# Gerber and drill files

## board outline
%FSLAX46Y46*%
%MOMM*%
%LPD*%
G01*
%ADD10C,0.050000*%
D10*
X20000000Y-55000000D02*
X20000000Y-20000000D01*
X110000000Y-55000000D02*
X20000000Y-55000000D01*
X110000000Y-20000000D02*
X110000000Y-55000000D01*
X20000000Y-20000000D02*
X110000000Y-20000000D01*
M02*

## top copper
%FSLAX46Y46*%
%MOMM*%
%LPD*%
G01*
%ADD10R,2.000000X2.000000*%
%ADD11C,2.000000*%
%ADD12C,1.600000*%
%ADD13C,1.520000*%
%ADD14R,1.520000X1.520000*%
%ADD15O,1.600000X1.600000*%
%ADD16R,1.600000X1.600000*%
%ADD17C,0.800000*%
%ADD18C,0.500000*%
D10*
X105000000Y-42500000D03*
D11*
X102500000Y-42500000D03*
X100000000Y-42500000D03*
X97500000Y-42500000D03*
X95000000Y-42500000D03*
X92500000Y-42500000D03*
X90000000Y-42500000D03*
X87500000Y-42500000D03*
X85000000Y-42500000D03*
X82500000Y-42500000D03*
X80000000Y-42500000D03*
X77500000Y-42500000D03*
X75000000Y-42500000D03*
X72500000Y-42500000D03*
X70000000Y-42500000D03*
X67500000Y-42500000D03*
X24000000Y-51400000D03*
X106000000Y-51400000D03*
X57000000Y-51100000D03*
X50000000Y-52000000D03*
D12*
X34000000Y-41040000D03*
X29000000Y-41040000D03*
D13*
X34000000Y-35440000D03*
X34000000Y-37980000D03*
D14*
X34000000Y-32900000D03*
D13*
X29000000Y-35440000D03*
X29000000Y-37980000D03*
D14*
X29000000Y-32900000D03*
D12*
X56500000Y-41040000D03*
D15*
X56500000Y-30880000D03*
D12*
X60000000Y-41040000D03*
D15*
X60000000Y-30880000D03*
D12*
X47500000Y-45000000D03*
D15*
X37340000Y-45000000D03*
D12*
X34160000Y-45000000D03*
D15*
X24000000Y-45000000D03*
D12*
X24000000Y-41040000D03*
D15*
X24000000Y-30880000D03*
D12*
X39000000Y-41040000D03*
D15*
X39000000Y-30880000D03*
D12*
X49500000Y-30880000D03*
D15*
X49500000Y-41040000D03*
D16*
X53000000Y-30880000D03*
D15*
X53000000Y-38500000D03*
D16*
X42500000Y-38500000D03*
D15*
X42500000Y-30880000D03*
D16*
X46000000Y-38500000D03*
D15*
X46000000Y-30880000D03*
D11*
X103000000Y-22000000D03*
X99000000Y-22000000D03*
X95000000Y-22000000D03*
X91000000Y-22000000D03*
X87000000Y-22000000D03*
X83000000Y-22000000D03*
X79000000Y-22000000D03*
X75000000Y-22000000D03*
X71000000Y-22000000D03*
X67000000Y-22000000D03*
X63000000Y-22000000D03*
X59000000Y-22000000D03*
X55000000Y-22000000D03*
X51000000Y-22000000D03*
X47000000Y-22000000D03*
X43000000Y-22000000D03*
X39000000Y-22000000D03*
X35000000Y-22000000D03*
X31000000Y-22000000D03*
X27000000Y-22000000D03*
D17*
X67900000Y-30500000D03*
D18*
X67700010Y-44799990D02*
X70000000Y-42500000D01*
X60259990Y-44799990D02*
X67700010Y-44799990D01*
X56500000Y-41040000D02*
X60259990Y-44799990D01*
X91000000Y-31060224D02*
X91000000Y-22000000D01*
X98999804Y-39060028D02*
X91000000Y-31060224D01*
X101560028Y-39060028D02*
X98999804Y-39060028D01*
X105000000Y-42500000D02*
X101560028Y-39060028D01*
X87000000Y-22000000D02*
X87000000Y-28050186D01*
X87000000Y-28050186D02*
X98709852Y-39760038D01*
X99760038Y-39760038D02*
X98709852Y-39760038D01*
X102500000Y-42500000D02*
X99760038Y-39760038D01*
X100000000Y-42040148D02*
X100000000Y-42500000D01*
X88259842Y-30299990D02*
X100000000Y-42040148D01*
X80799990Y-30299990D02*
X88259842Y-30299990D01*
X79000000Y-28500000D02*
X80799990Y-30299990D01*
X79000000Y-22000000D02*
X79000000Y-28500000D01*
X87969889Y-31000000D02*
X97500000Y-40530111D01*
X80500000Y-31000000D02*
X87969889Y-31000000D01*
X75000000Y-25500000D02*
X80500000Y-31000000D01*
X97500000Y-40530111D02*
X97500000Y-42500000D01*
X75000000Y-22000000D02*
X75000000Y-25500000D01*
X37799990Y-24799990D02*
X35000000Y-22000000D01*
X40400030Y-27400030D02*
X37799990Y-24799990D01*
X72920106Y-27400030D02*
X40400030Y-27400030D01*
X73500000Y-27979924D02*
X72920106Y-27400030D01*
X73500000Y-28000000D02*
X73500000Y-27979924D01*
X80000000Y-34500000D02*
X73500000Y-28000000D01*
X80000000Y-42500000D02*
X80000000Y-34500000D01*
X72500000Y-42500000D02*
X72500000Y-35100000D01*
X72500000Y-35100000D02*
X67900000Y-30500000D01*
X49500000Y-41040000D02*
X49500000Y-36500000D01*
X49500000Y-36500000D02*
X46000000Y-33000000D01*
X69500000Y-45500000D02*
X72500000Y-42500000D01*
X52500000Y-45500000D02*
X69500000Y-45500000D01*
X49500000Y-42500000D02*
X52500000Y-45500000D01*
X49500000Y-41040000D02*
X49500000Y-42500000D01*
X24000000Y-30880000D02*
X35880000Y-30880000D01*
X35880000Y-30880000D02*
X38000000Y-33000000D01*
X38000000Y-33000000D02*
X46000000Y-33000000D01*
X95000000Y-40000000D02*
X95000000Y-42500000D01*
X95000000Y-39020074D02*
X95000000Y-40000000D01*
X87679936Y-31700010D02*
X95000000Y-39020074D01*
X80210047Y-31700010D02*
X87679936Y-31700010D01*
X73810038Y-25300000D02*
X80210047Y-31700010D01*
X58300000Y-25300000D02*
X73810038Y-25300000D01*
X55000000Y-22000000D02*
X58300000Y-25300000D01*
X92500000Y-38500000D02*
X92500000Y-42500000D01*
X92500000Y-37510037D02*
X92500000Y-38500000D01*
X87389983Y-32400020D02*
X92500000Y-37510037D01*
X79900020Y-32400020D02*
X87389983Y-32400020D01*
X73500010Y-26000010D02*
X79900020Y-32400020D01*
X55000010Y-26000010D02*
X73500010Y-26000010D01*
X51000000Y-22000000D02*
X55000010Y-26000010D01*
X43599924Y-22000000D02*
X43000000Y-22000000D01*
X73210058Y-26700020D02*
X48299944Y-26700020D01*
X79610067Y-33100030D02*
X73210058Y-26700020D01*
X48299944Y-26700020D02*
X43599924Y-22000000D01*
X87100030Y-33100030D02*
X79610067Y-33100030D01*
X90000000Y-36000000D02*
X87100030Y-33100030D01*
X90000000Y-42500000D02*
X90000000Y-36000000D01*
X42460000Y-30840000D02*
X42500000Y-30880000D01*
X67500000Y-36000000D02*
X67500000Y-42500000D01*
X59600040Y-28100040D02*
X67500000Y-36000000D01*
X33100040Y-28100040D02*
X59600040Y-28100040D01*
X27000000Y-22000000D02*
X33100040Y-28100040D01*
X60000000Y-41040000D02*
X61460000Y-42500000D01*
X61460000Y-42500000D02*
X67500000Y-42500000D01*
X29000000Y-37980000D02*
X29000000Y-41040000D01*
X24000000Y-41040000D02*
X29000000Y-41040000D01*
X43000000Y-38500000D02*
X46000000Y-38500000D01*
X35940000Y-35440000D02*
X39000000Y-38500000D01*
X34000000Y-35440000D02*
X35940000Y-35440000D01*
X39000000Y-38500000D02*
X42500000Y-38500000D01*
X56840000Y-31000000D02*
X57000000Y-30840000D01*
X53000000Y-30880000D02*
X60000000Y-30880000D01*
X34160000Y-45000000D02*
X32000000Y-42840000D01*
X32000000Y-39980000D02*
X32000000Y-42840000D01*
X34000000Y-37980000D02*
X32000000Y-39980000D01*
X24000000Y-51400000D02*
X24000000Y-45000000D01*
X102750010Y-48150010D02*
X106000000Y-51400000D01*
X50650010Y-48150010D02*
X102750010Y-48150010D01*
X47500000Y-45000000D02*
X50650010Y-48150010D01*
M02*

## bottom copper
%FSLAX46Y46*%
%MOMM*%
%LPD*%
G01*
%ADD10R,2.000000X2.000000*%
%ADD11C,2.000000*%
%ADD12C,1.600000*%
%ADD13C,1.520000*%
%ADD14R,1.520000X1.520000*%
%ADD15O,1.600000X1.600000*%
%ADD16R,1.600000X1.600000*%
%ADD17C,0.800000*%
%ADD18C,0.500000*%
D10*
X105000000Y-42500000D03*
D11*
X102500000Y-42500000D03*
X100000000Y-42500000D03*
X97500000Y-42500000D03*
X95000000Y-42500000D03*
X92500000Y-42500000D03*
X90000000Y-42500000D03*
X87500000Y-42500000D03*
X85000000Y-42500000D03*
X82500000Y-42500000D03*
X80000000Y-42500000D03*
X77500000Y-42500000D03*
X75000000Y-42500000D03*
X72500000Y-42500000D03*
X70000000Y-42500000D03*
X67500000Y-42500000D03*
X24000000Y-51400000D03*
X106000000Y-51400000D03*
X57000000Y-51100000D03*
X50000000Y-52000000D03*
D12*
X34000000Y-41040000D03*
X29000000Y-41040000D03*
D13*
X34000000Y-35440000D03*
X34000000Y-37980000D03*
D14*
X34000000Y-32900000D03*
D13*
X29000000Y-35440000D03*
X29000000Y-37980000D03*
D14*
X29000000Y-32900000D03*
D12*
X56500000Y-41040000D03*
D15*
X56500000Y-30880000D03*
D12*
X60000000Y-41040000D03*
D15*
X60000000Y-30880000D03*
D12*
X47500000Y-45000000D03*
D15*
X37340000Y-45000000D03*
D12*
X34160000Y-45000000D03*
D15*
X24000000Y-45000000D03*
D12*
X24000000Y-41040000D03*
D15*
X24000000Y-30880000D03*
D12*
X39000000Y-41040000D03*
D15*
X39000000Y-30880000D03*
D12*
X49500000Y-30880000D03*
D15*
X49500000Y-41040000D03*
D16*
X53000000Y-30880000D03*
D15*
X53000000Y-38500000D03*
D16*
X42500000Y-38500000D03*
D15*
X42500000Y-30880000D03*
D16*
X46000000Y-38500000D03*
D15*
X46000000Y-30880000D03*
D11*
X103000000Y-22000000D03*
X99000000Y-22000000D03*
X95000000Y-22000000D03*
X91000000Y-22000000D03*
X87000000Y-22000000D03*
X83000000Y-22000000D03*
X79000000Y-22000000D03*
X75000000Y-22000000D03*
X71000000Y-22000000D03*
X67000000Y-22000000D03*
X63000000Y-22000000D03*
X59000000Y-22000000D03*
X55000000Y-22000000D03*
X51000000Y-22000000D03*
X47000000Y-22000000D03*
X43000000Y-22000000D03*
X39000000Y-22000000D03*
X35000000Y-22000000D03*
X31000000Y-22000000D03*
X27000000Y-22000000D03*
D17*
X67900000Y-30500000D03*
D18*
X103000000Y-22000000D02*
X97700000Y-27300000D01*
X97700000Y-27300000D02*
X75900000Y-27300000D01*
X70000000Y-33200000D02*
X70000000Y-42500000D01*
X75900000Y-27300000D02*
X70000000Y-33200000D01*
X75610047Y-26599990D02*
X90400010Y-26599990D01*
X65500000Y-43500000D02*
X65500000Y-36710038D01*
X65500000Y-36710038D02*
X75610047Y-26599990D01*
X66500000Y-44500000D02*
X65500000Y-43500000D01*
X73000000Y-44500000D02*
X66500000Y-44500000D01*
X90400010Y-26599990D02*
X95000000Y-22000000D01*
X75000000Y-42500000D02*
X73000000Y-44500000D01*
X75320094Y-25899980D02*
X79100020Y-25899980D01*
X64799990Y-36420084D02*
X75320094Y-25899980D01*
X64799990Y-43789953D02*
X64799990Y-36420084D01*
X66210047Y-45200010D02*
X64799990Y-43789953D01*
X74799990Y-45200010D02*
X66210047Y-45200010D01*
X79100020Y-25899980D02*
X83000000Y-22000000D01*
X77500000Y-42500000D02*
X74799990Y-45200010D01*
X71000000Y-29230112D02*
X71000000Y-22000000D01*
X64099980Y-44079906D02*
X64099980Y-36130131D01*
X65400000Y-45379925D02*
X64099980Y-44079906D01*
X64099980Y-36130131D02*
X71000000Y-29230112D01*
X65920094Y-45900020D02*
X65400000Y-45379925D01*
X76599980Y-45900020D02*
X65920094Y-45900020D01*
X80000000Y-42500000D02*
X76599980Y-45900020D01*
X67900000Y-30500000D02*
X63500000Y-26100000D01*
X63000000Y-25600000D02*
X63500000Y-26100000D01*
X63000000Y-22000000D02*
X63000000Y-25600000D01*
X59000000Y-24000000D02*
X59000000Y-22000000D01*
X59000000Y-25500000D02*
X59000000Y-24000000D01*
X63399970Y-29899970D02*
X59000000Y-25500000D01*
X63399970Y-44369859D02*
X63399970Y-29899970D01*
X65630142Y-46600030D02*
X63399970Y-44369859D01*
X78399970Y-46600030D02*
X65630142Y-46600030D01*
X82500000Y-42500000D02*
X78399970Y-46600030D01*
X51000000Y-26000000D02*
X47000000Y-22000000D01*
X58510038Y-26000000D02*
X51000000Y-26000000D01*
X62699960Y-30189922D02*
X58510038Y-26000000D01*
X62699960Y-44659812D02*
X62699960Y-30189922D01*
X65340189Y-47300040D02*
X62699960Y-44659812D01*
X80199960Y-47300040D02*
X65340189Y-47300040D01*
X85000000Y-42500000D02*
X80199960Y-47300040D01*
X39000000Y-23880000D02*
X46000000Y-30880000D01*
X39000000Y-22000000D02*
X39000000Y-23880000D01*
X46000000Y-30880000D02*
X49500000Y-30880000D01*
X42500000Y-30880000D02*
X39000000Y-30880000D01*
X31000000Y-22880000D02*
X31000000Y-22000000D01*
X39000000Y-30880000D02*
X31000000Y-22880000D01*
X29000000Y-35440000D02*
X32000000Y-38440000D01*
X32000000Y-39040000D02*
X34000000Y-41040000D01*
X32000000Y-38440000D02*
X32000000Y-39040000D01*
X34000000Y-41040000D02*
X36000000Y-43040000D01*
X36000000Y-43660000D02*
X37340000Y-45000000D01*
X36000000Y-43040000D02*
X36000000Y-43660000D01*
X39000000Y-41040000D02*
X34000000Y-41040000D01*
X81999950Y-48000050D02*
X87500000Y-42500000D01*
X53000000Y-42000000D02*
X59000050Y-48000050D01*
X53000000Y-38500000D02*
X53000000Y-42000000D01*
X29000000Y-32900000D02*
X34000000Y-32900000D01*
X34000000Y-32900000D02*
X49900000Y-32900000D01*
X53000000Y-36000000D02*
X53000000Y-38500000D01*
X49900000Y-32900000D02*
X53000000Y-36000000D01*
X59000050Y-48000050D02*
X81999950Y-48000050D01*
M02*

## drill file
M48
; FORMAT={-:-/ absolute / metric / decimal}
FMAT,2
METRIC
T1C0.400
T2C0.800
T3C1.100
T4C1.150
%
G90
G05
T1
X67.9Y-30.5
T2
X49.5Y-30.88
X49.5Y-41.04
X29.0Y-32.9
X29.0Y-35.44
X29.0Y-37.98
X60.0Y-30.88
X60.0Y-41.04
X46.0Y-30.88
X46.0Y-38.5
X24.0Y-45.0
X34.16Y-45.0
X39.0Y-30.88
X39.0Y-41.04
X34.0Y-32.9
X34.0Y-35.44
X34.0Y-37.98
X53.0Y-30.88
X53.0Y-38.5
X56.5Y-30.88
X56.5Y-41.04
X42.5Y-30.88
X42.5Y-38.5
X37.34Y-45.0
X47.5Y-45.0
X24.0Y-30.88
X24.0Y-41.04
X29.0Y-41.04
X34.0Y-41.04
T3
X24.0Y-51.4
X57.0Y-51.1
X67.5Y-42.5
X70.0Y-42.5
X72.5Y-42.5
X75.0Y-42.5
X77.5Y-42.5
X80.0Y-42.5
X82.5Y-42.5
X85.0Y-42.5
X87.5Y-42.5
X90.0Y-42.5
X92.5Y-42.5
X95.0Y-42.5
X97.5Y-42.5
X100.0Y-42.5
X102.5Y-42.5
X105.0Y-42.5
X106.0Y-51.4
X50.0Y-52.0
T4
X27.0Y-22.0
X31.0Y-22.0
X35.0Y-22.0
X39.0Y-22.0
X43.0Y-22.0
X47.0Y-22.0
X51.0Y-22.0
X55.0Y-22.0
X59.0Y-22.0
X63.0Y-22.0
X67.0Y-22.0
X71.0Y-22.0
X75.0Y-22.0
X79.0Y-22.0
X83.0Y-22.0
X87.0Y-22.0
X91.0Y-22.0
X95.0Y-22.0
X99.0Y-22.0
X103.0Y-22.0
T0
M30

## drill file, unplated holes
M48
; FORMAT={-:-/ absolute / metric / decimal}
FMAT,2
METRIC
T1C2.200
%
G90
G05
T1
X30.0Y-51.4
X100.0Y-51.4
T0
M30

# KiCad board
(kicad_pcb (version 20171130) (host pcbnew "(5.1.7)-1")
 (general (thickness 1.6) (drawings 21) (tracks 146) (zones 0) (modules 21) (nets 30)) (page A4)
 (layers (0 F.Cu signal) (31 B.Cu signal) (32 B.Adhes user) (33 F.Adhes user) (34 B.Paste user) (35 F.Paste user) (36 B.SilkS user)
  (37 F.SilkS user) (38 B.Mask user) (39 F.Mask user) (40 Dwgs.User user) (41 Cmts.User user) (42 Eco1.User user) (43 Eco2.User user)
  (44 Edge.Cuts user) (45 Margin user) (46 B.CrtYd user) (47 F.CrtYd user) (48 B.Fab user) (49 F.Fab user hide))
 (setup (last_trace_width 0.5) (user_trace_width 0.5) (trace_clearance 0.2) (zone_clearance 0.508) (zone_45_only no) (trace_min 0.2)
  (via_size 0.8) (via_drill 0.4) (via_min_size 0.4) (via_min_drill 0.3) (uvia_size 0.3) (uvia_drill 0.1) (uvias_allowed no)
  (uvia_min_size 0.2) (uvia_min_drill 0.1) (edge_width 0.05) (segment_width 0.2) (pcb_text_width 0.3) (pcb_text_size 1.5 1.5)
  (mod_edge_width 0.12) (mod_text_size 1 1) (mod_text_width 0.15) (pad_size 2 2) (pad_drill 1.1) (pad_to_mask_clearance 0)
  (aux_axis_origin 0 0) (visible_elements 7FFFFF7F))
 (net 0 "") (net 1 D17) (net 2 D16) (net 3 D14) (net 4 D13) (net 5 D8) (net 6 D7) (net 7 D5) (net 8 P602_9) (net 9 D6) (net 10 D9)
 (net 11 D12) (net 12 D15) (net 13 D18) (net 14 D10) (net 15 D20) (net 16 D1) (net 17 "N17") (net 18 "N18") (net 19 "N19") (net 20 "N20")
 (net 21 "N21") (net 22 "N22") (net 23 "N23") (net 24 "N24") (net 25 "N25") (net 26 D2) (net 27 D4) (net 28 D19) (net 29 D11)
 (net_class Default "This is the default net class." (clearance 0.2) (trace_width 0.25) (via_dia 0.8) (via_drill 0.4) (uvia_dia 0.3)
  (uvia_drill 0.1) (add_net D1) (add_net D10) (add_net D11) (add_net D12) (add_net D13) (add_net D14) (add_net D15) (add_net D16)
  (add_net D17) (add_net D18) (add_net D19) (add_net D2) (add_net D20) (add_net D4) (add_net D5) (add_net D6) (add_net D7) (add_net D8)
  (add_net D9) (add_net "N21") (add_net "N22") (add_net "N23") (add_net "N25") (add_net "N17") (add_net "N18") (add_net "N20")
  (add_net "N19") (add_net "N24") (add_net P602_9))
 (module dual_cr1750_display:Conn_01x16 (layer F.Cu) (at 105 42.5 180) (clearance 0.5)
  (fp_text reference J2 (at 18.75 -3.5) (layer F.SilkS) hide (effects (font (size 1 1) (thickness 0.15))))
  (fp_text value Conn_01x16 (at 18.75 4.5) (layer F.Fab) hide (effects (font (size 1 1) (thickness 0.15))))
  (pad 1 thru_hole rect (at 0 0 180) (size 2 2) (drill 1.1) (layers *.Cu *.Mask) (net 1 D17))
  (pad 2 thru_hole circle (at 2.5 0 180) (size 2 2) (drill 1.1) (layers *.Cu *.Mask) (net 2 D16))
  (pad 3 thru_hole circle (at 5 0 180) (size 2 2) (drill 1.1) (layers *.Cu *.Mask) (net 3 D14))
  (pad 4 thru_hole circle (at 7.5 0 180) (size 2 2) (drill 1.1) (layers *.Cu *.Mask) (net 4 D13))
  (pad 5 thru_hole circle (at 10 0 180) (size 2 2) (drill 1.1) (layers *.Cu *.Mask) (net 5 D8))
  (pad 6 thru_hole circle (at 12.5 0 180) (size 2 2) (drill 1.1) (layers *.Cu *.Mask) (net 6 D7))
  (pad 7 thru_hole circle (at 15 0 180) (size 2 2) (drill 1.1) (layers *.Cu *.Mask) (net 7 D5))
  (pad 8 thru_hole circle (at 17.5 0 180) (size 2 2) (drill 1.1) (layers *.Cu *.Mask) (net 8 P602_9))
  (pad 9 thru_hole circle (at 20 0 180) (size 2 2) (drill 1.1) (layers *.Cu *.Mask) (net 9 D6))
  (pad 10 thru_hole circle (at 22.5 0 180) (size 2 2) (drill 1.1) (layers *.Cu *.Mask) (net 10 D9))
  (pad 11 thru_hole circle (at 25 0 180) (size 2 2) (drill 1.1) (layers *.Cu *.Mask) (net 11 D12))
  (pad 12 thru_hole circle (at 27.5 0 180) (size 2 2) (drill 1.1) (layers *.Cu *.Mask) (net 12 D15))
  (pad 13 thru_hole circle (at 30 0 180) (size 2 2) (drill 1.1) (layers *.Cu *.Mask) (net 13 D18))
  (pad 14 thru_hole circle (at 32.5 0 180) (size 2 2) (drill 1.1) (layers *.Cu *.Mask) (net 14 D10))
  (pad 15 thru_hole circle (at 35 0 180) (size 2 2) (drill 1.1) (layers *.Cu *.Mask) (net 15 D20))
  (pad 16 thru_hole circle (at 37.5 0 180) (size 2 2) (drill 1.1) (layers *.Cu *.Mask) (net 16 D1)))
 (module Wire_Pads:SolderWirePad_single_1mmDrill (layer F.Cu) (at 24 51.4)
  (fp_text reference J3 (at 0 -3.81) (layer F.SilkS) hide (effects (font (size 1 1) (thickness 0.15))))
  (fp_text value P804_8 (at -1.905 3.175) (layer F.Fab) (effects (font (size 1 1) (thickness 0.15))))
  (pad 1 thru_hole circle (at 0 0) (size 2 2) (drill 1.1) (layers *.Cu *.Mask) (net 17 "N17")))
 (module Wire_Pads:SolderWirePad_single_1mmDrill (layer F.Cu) (at 106 51.4)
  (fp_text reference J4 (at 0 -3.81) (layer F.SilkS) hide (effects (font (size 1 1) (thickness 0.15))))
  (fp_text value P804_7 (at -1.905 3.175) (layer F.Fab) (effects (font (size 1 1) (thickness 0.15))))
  (pad 1 thru_hole circle (at 0 0) (size 2 2) (drill 1.1) (layers *.Cu *.Mask) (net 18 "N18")))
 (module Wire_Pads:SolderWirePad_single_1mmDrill (layer F.Cu) (at 57 51.1)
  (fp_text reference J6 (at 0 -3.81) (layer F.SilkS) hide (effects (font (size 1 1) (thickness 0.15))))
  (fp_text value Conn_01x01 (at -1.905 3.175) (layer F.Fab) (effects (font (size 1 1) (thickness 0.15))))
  (pad 1 thru_hole circle (at 0 0) (size 2 2) (drill 1.1) (layers *.Cu *.Mask) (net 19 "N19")))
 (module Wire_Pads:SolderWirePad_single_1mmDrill (layer F.Cu) (at 50 52)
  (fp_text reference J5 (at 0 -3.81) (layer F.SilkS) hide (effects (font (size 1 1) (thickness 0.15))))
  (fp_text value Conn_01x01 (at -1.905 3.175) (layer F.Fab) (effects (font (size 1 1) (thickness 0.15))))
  (pad 1 thru_hole circle (at 0 0) (size 2 2) (drill 1.1) (layers *.Cu *.Mask) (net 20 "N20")))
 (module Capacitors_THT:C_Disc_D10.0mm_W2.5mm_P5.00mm (layer F.Cu) (at 34 41.04 180)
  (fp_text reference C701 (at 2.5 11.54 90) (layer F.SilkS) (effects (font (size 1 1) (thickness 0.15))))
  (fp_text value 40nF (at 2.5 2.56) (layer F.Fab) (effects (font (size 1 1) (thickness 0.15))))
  (pad 1 thru_hole circle (at 0 0 180) (size 1.6 1.6) (drill 0.8) (layers *.Cu *.Mask) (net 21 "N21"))
  (pad 2 thru_hole circle (at 5 0 180) (size 1.6 1.6) (drill 0.8) (layers *.Cu *.Mask) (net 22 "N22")))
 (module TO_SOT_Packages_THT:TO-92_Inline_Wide (layer F.Cu) (at 34 32.9 270)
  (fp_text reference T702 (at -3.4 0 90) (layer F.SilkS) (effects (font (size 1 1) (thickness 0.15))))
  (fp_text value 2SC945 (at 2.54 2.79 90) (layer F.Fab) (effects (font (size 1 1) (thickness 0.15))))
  (pad 2 thru_hole circle (at 2.54 0) (size 1.52 1.52) (drill 0.8) (layers *.Cu *.Mask) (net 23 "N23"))
  (pad 3 thru_hole circle (at 5.08 0) (size 1.52 1.52) (drill 0.8) (layers *.Cu *.Mask) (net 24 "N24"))
  (pad 1 thru_hole rect (at 0 0) (size 1.52 1.52) (drill 0.8) (layers *.Cu *.Mask) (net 8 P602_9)))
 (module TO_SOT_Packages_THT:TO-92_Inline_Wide (layer F.Cu) (at 29 32.9 270)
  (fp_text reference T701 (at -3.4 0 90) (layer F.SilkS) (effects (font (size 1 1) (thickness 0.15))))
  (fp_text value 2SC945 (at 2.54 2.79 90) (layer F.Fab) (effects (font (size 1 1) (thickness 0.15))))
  (pad 2 thru_hole circle (at 2.54 0) (size 1.52 1.52) (drill 0.8) (layers *.Cu *.Mask) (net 21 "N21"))
  (pad 3 thru_hole circle (at 5.08 0) (size 1.52 1.52) (drill 0.8) (layers *.Cu *.Mask) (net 22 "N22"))
  (pad 1 thru_hole rect (at 0 0) (size 1.52 1.52) (drill 0.8) (layers *.Cu *.Mask) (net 8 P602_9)))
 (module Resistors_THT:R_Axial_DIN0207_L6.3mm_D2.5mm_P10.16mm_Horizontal (layer F.Cu) (at 56.5 41.04 90)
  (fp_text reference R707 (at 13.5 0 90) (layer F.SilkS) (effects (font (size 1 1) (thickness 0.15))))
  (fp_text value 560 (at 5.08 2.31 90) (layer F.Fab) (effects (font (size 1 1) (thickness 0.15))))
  (pad 1 thru_hole circle (at 0 0 90) (size 1.6 1.6) (drill 0.8) (layers *.Cu *.Mask) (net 15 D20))
  (pad 2 thru_hole oval (at 10.16 0 90) (size 1.6 1.6) (drill 0.8) (layers *.Cu *.Mask) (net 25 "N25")))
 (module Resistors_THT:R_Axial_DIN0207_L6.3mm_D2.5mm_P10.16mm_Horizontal (layer F.Cu) (at 60 41.04 90)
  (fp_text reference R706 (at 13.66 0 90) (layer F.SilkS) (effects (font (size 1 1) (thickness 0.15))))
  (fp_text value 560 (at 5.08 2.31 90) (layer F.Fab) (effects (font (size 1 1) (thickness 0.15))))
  (pad 1 thru_hole circle (at 0 0 90) (size 1.6 1.6) (drill 0.8) (layers *.Cu *.Mask) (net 16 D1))
  (pad 2 thru_hole oval (at 10.16 0 90) (size 1.6 1.6) (drill 0.8) (layers *.Cu *.Mask) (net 25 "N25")))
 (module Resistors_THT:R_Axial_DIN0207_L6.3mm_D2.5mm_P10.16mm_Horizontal (layer F.Cu) (at 47.5 45 180)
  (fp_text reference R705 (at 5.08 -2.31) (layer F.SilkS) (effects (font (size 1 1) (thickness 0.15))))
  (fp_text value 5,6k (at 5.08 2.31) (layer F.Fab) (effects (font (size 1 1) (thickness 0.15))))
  (pad 1 thru_hole circle (at 0 0 180) (size 1.6 1.6) (drill 0.8) (layers *.Cu *.Mask) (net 18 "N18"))
  (pad 2 thru_hole oval (at 10.16 0 180) (size 1.6 1.6) (drill 0.8) (layers *.Cu *.Mask) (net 21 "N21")))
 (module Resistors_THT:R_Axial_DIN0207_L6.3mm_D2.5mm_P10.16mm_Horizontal (layer F.Cu) (at 34.16 45 180)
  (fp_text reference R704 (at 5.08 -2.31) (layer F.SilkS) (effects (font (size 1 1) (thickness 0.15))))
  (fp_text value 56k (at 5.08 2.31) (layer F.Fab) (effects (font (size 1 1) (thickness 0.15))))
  (pad 1 thru_hole circle (at 0 0 180) (size 1.6 1.6) (drill 0.8) (layers *.Cu *.Mask) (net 24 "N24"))
  (pad 2 thru_hole oval (at 10.16 0 180) (size 1.6 1.6) (drill 0.8) (layers *.Cu *.Mask) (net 17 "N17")))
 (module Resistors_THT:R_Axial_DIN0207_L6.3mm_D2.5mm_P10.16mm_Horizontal (layer F.Cu) (at 24 41.04 90)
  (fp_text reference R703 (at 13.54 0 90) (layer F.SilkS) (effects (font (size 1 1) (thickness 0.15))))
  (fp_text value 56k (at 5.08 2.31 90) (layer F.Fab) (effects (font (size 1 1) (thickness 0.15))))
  (pad 1 thru_hole circle (at 0 0 90) (size 1.6 1.6) (drill 0.8) (layers *.Cu *.Mask) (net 22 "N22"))
  (pad 2 thru_hole oval (at 10.16 0 90) (size 1.6 1.6) (drill 0.8) (layers *.Cu *.Mask) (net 14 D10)))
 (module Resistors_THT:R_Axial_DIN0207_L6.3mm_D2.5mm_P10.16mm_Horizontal (layer F.Cu) (at 39 41.04 90)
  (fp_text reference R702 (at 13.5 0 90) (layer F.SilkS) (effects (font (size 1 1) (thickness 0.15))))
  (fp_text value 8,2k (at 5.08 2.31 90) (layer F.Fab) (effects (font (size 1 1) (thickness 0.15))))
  (pad 1 thru_hole circle (at 0 0 90) (size 1.6 1.6) (drill 0.8) (layers *.Cu *.Mask) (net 21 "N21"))
  (pad 2 thru_hole oval (at 10.16 0 90) (size 1.6 1.6) (drill 0.8) (layers *.Cu *.Mask) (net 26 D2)))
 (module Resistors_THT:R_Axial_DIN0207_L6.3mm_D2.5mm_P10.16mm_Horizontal (layer F.Cu) (at 49.5 30.88 270)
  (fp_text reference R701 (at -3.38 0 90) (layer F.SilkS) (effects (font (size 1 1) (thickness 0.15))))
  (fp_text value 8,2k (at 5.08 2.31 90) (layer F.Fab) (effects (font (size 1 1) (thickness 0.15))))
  (pad 1 thru_hole circle (at 0 0 270) (size 1.6 1.6) (drill 0.8) (layers *.Cu *.Mask) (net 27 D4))
  (pad 2 thru_hole oval (at 10.16 0 270) (size 1.6 1.6) (drill 0.8) (layers *.Cu *.Mask) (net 14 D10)))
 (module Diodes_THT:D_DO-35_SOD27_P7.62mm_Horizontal (layer F.Cu) (at 53 30.88 270)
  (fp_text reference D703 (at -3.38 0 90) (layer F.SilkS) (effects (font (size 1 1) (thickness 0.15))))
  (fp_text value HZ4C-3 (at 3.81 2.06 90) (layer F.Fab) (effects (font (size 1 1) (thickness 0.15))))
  (pad 1 thru_hole rect (at 0 0 270) (size 1.6 1.6) (drill 0.8) (layers *.Cu *.Mask) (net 25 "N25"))
  (pad 2 thru_hole oval (at 7.62 0 270) (size 1.6 1.6) (drill 0.8) (layers *.Cu *.Mask) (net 8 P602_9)))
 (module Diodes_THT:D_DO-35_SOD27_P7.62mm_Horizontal (layer F.Cu) (at 42.5 38.5 90)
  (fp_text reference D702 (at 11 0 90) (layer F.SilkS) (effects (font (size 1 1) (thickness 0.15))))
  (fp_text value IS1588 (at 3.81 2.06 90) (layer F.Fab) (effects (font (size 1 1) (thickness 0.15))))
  (pad 1 thru_hole rect (at 0 0 90) (size 1.6 1.6) (drill 0.8) (layers *.Cu *.Mask) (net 23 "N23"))
  (pad 2 thru_hole oval (at 7.62 0 90) (size 1.6 1.6) (drill 0.8) (layers *.Cu *.Mask) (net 26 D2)))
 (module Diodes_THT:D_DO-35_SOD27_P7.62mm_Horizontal (layer F.Cu) (at 46 38.5 90)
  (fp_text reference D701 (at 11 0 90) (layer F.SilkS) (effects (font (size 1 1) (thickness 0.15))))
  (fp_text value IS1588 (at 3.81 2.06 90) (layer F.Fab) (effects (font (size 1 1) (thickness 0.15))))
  (pad 1 thru_hole rect (at 0 0 90) (size 1.6 1.6) (drill 0.8) (layers *.Cu *.Mask) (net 23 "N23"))
  (pad 2 thru_hole oval (at 7.62 0 90) (size 1.6 1.6) (drill 0.8) (layers *.Cu *.Mask) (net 27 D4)))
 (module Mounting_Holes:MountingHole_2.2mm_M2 (layer F.Cu) (at 100 51.4)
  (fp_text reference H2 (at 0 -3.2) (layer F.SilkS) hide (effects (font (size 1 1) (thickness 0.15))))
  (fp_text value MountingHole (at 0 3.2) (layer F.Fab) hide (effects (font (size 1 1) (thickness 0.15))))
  (pad 1 np_thru_hole circle (at 0 0) (size 2.2 2.2) (drill 2.2) (layers *.Cu *.Mask)))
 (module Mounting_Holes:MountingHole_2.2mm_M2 (layer F.Cu) (at 30 51.4)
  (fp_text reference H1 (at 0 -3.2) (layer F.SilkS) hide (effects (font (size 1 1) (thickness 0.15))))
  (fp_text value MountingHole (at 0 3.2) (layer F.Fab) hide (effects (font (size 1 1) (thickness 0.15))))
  (pad 1 np_thru_hole circle (at 0 0) (size 2.2 2.2) (drill 2.2) (layers *.Cu *.Mask)))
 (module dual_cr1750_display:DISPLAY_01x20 (layer F.Cu) (at 27 22)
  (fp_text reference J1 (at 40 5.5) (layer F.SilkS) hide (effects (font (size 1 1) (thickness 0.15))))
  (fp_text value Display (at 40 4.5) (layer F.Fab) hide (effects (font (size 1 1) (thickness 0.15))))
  (pad 20 thru_hole circle (at 76 0) (size 2 2) (drill 1.15) (layers *.Cu *.Mask) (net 15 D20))
  (pad 19 thru_hole circle (at 72 0) (size 2 2) (drill 1.15) (layers *.Cu *.Mask) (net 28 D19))
  (pad 18 thru_hole circle (at 68 0) (size 2 2) (drill 1.15) (layers *.Cu *.Mask) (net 13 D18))
  (pad 17 thru_hole circle (at 64 0) (size 2 2) (drill 1.15) (layers *.Cu *.Mask) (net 1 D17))
  (pad 16 thru_hole circle (at 60 0) (size 2 2) (drill 1.15) (layers *.Cu *.Mask) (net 2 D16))
  (pad 15 thru_hole circle (at 56 0) (size 2 2) (drill 1.15) (layers *.Cu *.Mask) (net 12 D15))
  (pad 14 thru_hole circle (at 52 0) (size 2 2) (drill 1.15) (layers *.Cu *.Mask) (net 3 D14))
  (pad 13 thru_hole circle (at 48 0) (size 2 2) (drill 1.15) (layers *.Cu *.Mask) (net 4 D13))
  (pad 12 thru_hole circle (at 44 0) (size 2 2) (drill 1.15) (layers *.Cu *.Mask) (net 11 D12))
  (pad 11 thru_hole circle (at 40 0) (size 2 2) (drill 1.15) (layers *.Cu *.Mask) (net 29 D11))
  (pad 10 thru_hole circle (at 36 0) (size 2 2) (drill 1.15) (layers *.Cu *.Mask) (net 14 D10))
  (pad 9 thru_hole circle (at 32 0) (size 2 2) (drill 1.15) (layers *.Cu *.Mask) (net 10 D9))
  (pad 8 thru_hole circle (at 28 0) (size 2 2) (drill 1.15) (layers *.Cu *.Mask) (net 5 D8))
  (pad 7 thru_hole circle (at 24 0) (size 2 2) (drill 1.15) (layers *.Cu *.Mask) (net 6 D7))
  (pad 6 thru_hole circle (at 20 0) (size 2 2) (drill 1.15) (layers *.Cu *.Mask) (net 9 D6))
  (pad 5 thru_hole circle (at 16 0) (size 2 2) (drill 1.15) (layers *.Cu *.Mask) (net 7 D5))
  (pad 4 thru_hole circle (at 12 0) (size 2 2) (drill 1.15) (layers *.Cu *.Mask) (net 27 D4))
  (pad 3 thru_hole circle (at 8 0) (size 2 2) (drill 1.15) (layers *.Cu *.Mask) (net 11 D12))
  (pad 2 thru_hole circle (at 4 0) (size 2 2) (drill 1.15) (layers *.Cu *.Mask) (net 26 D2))
  (pad 1 thru_hole circle (at 0 0) (size 2 2) (drill 1.15) (layers *.Cu *.Mask) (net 16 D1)))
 (gr_line (start 20 55) (end 20 20) (layer Edge.Cuts) (width 0.05))
 (gr_line (start 110 55) (end 20 55) (layer Edge.Cuts) (width 0.05))
 (gr_line (start 110 20) (end 110 55) (layer Edge.Cuts) (width 0.05))
 (gr_line (start 20 20) (end 110 20) (layer Edge.Cuts) (width 0.05))
 (segment (start 103 22) (end 97.7 27.3) (width 0.5) (layer B.Cu) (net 15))
 (segment (start 97.7 27.3) (end 75.9 27.3) (width 0.5) (layer B.Cu) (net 15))
 (segment (start 70 33.2) (end 70 42.5) (width 0.5) (layer B.Cu) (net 15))
 (segment (start 75.9 27.3) (end 70 33.2) (width 0.5) (layer B.Cu) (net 15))
 (segment (start 67.70001 44.79999) (end 70 42.5) (width 0.5) (layer F.Cu) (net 15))
 (segment (start 60.25999 44.79999) (end 67.70001 44.79999) (width 0.5) (layer F.Cu) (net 15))
 (segment (start 56.5 41.04) (end 60.25999 44.79999) (width 0.5) (layer F.Cu) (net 15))
 (segment (start 75.610047 26.59999) (end 90.40001 26.59999) (width 0.5) (layer B.Cu) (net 13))
 (segment (start 65.5 43.5) (end 65.5 36.710038) (width 0.5) (layer B.Cu) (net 13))
 (segment (start 65.5 36.710038) (end 75.610047 26.59999) (width 0.5) (layer B.Cu) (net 13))
 (segment (start 66.5 44.5) (end 65.5 43.5) (width 0.5) (layer B.Cu) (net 13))
 (segment (start 73 44.5) (end 66.5 44.5) (width 0.5) (layer B.Cu) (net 13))
 (segment (start 90.40001 26.59999) (end 95 22) (width 0.5) (layer B.Cu) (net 13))
 (segment (start 75 42.5) (end 73 44.5) (width 0.5) (layer B.Cu) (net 13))
 (segment (start 91 31.060224) (end 91 22) (width 0.5) (layer F.Cu) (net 1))
 (segment (start 98.999804 39.060028) (end 91 31.060224) (width 0.5) (layer F.Cu) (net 1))
 (segment (start 101.560028 39.060028) (end 98.999804 39.060028) (width 0.5) (layer F.Cu) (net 1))
 (segment (start 105 42.5) (end 101.560028 39.060028) (width 0.5) (layer F.Cu) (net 1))
 (segment (start 87 22) (end 87 28.050186) (width 0.5) (layer F.Cu) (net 2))
 (segment (start 87 28.050186) (end 98.709852 39.760038) (width 0.5) (layer F.Cu) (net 2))
 (segment (start 99.760038 39.760038) (end 98.709852 39.760038) (width 0.5) (layer F.Cu) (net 2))
 (segment (start 102.5 42.5) (end 99.760038 39.760038) (width 0.5) (layer F.Cu) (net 2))
 (segment (start 75.320094 25.89998) (end 79.10002 25.89998) (width 0.5) (layer B.Cu) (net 12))
 (segment (start 64.79999 36.420084) (end 75.320094 25.89998) (width 0.5) (layer B.Cu) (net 12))
 (segment (start 64.79999 43.789953) (end 64.79999 36.420084) (width 0.5) (layer B.Cu) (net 12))
 (segment (start 66.210047 45.20001) (end 64.79999 43.789953) (width 0.5) (layer B.Cu) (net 12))
 (segment (start 74.79999 45.20001) (end 66.210047 45.20001) (width 0.5) (layer B.Cu) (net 12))
 (segment (start 79.10002 25.89998) (end 83 22) (width 0.5) (layer B.Cu) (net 12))
 (segment (start 77.5 42.5) (end 74.79999 45.20001) (width 0.5) (layer B.Cu) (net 12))
 (segment (start 100 42.040148) (end 100 42.5) (width 0.5) (layer F.Cu) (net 3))
 (segment (start 88.259842 30.29999) (end 100 42.040148) (width 0.5) (layer F.Cu) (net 3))
 (segment (start 80.79999 30.29999) (end 88.259842 30.29999) (width 0.5) (layer F.Cu) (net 3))
 (segment (start 79 28.5) (end 80.79999 30.29999) (width 0.5) (layer F.Cu) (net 3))
 (segment (start 79 22) (end 79 28.5) (width 0.5) (layer F.Cu) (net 3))
 (segment (start 87.969889 31) (end 97.5 40.530111) (width 0.5) (layer F.Cu) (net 4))
 (segment (start 80.5 31) (end 87.969889 31) (width 0.5) (layer F.Cu) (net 4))
 (segment (start 75 25.5) (end 80.5 31) (width 0.5) (layer F.Cu) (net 4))
 (segment (start 97.5 40.530111) (end 97.5 42.5) (width 0.5) (layer F.Cu) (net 4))
 (segment (start 75 22) (end 75 25.5) (width 0.5) (layer F.Cu) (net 4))
 (segment (start 71 29.230112) (end 71 22) (width 0.5) (layer B.Cu) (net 11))
 (segment (start 64.09998 44.079906) (end 64.09998 36.130131) (width 0.5) (layer B.Cu) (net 11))
 (segment (start 65.4 45.379925) (end 64.09998 44.079906) (width 0.5) (layer B.Cu) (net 11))
 (segment (start 64.09998 36.130131) (end 71 29.230112) (width 0.5) (layer B.Cu) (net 11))
 (segment (start 65.920094 45.90002) (end 65.4 45.379925) (width 0.5) (layer B.Cu) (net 11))
 (segment (start 76.59998 45.90002) (end 65.920094 45.90002) (width 0.5) (layer B.Cu) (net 11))
 (segment (start 80 42.5) (end 76.59998 45.90002) (width 0.5) (layer B.Cu) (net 11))
 (segment (start 37.79999 24.79999) (end 35 22) (width 0.5) (layer F.Cu) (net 11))
 (segment (start 40.40003 27.40003) (end 37.79999 24.79999) (width 0.5) (layer F.Cu) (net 11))
 (segment (start 72.920106 27.40003) (end 40.40003 27.40003) (width 0.5) (layer F.Cu) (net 11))
 (segment (start 73.5 27.979924) (end 72.920106 27.40003) (width 0.5) (layer F.Cu) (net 11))
 (segment (start 73.5 28) (end 73.5 27.979924) (width 0.5) (layer F.Cu) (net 11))
 (segment (start 80 34.5) (end 73.5 28) (width 0.5) (layer F.Cu) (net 11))
 (segment (start 80 42.5) (end 80 34.5) (width 0.5) (layer F.Cu) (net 11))
 (segment (start 72.5 42.5) (end 72.5 35.1) (width 0.5) (layer F.Cu) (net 14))
 (segment (start 72.5 35.1) (end 67.9 30.5) (width 0.5) (layer F.Cu) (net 14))
 (via (at 67.9 30.5) (size 0.8) (drill 0.4) (layers F.Cu B.Cu) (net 14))
 (segment (start 67.9 30.5) (end 63.5 26.1) (width 0.5) (layer B.Cu) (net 14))
 (segment (start 63 25.6) (end 63.5 26.1) (width 0.5) (layer B.Cu) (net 14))
 (segment (start 63 22) (end 63 25.6) (width 0.5) (layer B.Cu) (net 14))
 (segment (start 49.5 41.04) (end 49.5 36.5) (width 0.5) (layer F.Cu) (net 14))
 (segment (start 49.5 36.5) (end 46 33) (width 0.5) (layer F.Cu) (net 14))
 (segment (start 69.5 45.5) (end 72.5 42.5) (width 0.5) (layer F.Cu) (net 14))
 (segment (start 52.5 45.5) (end 69.5 45.5) (width 0.5) (layer F.Cu) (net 14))
 (segment (start 49.5 42.5) (end 52.5 45.5) (width 0.5) (layer F.Cu) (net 14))
 (segment (start 49.5 41.04) (end 49.5 42.5) (width 0.5) (layer F.Cu) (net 14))
 (segment (start 24 30.88) (end 35.88 30.88) (width 0.5) (layer F.Cu) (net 14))
 (segment (start 35.88 30.88) (end 38 33) (width 0.5) (layer F.Cu) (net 14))
 (segment (start 38 33) (end 46 33) (width 0.5) (layer F.Cu) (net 14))
 (segment (start 59 24) (end 59 22) (width 0.5) (layer B.Cu) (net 10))
 (segment (start 59 25.5) (end 59 24) (width 0.5) (layer B.Cu) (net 10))
 (segment (start 63.39997 29.89997) (end 59 25.5) (width 0.5) (layer B.Cu) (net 10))
 (segment (start 63.39997 44.369859) (end 63.39997 29.89997) (width 0.5) (layer B.Cu) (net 10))
 (segment (start 65.630142 46.60003) (end 63.39997 44.369859) (width 0.5) (layer B.Cu) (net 10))
 (segment (start 78.39997 46.60003) (end 65.630142 46.60003) (width 0.5) (layer B.Cu) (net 10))
 (segment (start 82.5 42.5) (end 78.39997 46.60003) (width 0.5) (layer B.Cu) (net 10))
 (segment (start 95 40) (end 95 42.5) (width 0.5) (layer F.Cu) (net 5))
 (segment (start 95 39.020074) (end 95 40) (width 0.5) (layer F.Cu) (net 5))
 (segment (start 87.679936 31.70001) (end 95 39.020074) (width 0.5) (layer F.Cu) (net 5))
 (segment (start 80.210047 31.70001) (end 87.679936 31.70001) (width 0.5) (layer F.Cu) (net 5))
 (segment (start 73.810038 25.3) (end 80.210047 31.70001) (width 0.5) (layer F.Cu) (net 5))
 (segment (start 58.3 25.3) (end 73.810038 25.3) (width 0.5) (layer F.Cu) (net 5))
 (segment (start 55 22) (end 58.3 25.3) (width 0.5) (layer F.Cu) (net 5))
 (segment (start 92.5 38.5) (end 92.5 42.5) (width 0.5) (layer F.Cu) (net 6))
 (segment (start 92.5 37.510037) (end 92.5 38.5) (width 0.5) (layer F.Cu) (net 6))
 (segment (start 87.389983 32.40002) (end 92.5 37.510037) (width 0.5) (layer F.Cu) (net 6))
 (segment (start 79.90002 32.40002) (end 87.389983 32.40002) (width 0.5) (layer F.Cu) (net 6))
 (segment (start 73.50001 26.00001) (end 79.90002 32.40002) (width 0.5) (layer F.Cu) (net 6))
 (segment (start 55.00001 26.00001) (end 73.50001 26.00001) (width 0.5) (layer F.Cu) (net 6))
 (segment (start 51 22) (end 55.00001 26.00001) (width 0.5) (layer F.Cu) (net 6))
 (segment (start 51 26) (end 47 22) (width 0.5) (layer B.Cu) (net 9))
 (segment (start 58.510038 26) (end 51 26) (width 0.5) (layer B.Cu) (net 9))
 (segment (start 62.69996 30.189922) (end 58.510038 26) (width 0.5) (layer B.Cu) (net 9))
 (segment (start 62.69996 44.659812) (end 62.69996 30.189922) (width 0.5) (layer B.Cu) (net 9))
 (segment (start 65.340189 47.30004) (end 62.69996 44.659812) (width 0.5) (layer B.Cu) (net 9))
 (segment (start 80.19996 47.30004) (end 65.340189 47.30004) (width 0.5) (layer B.Cu) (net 9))
 (segment (start 85 42.5) (end 80.19996 47.30004) (width 0.5) (layer B.Cu) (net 9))
 (segment (start 43.599924 22) (end 43 22) (width 0.5) (layer F.Cu) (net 7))
 (segment (start 73.210058 26.70002) (end 48.299944 26.70002) (width 0.5) (layer F.Cu) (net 7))
 (segment (start 79.610067 33.10003) (end 73.210058 26.70002) (width 0.5) (layer F.Cu) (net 7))
 (segment (start 48.299944 26.70002) (end 43.599924 22) (width 0.5) (layer F.Cu) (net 7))
 (segment (start 87.10003 33.10003) (end 79.610067 33.10003) (width 0.5) (layer F.Cu) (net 7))
 (segment (start 90 36) (end 87.10003 33.10003) (width 0.5) (layer F.Cu) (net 7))
 (segment (start 90 42.5) (end 90 36) (width 0.5) (layer F.Cu) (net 7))
 (segment (start 39 23.88) (end 46 30.88) (width 0.5) (layer B.Cu) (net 27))
 (segment (start 39 22) (end 39 23.88) (width 0.5) (layer B.Cu) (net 27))
 (segment (start 46 30.88) (end 49.5 30.88) (width 0.5) (layer B.Cu) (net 27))
 (segment (start 42.46 30.84) (end 42.5 30.88) (width 0.5) (layer F.Cu) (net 26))
 (segment (start 42.5 30.88) (end 39 30.88) (width 0.5) (layer B.Cu) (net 26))
 (segment (start 31 22.88) (end 31 22) (width 0.5) (layer B.Cu) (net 26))
 (segment (start 39 30.88) (end 31 22.88) (width 0.5) (layer B.Cu) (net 26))
 (segment (start 67.5 36) (end 67.5 42.5) (width 0.5) (layer F.Cu) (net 16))
 (segment (start 59.60004 28.10004) (end 67.5 36) (width 0.5) (layer F.Cu) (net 16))
 (segment (start 33.10004 28.10004) (end 59.60004 28.10004) (width 0.5) (layer F.Cu) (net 16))
 (segment (start 27 22) (end 33.10004 28.10004) (width 0.5) (layer F.Cu) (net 16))
 (segment (start 60 41.04) (end 61.46 42.5) (width 0.5) (layer F.Cu) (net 16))
 (segment (start 61.46 42.5) (end 67.5 42.5) (width 0.5) (layer F.Cu) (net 16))
 (segment (start 29 35.44) (end 32 38.44) (width 0.5) (layer B.Cu) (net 21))
 (segment (start 32 39.04) (end 34 41.04) (width 0.5) (layer B.Cu) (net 21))
 (segment (start 32 38.44) (end 32 39.04) (width 0.5) (layer B.Cu) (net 21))
 (segment (start 34 41.04) (end 36 43.04) (width 0.5) (layer B.Cu) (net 21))
 (segment (start 36 43.66) (end 37.34 45) (width 0.5) (layer B.Cu) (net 21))
 (segment (start 36 43.04) (end 36 43.66) (width 0.5) (layer B.Cu) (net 21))
 (segment (start 39 41.04) (end 34 41.04) (width 0.5) (layer B.Cu) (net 21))
 (segment (start 29 37.98) (end 29 41.04) (width 0.5) (layer F.Cu) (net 22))
 (segment (start 24 41.04) (end 29 41.04) (width 0.5) (layer F.Cu) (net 22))
 (segment (start 43 38.5) (end 46 38.5) (width 0.5) (layer F.Cu) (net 23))
 (segment (start 35.94 35.44) (end 39 38.5) (width 0.5) (layer F.Cu) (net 23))
 (segment (start 34 35.44) (end 35.94 35.44) (width 0.5) (layer F.Cu) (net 23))
 (segment (start 39 38.5) (end 42.5 38.5) (width 0.5) (layer F.Cu) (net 23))
 (segment (start 56.84 31) (end 57 30.84) (width 0.5) (layer F.Cu) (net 25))
 (segment (start 53 30.88) (end 60 30.88) (width 0.5) (layer F.Cu) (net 25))
 (segment (start 34.16 45) (end 32 42.84) (width 0.5) (layer F.Cu) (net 24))
 (segment (start 32 39.98) (end 32 42.84) (width 0.5) (layer F.Cu) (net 24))
 (segment (start 34 37.98) (end 32 39.98) (width 0.5) (layer F.Cu) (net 24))
 (segment (start 81.99995 48.00005) (end 87.5 42.5) (width 0.5) (layer B.Cu) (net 8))
 (segment (start 53 42) (end 59.00005 48.00005) (width 0.5) (layer B.Cu) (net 8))
 (segment (start 53 38.5) (end 53 42) (width 0.5) (layer B.Cu) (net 8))
 (segment (start 29 32.9) (end 34 32.9) (width 0.5) (layer B.Cu) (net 8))
 (segment (start 34 32.9) (end 49.9 32.9) (width 0.5) (layer B.Cu) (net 8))
 (segment (start 53 36) (end 53 38.5) (width 0.5) (layer B.Cu) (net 8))
 (segment (start 49.9 32.9) (end 53 36) (width 0.5) (layer B.Cu) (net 8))
 (segment (start 59.00005 48.00005) (end 81.99995 48.00005) (width 0.5) (layer B.Cu) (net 8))
 (segment (start 24 51.4) (end 24 45) (width 0.5) (layer F.Cu) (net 17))
 (segment (start 102.75001 48.15001) (end 106 51.4) (width 0.5) (layer F.Cu) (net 18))
 (segment (start 50.65001 48.15001) (end 102.75001 48.15001) (width 0.5) (layer F.Cu) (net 18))
 (segment (start 47.5 45) (end 50.65001 48.15001) (width 0.5) (layer F.Cu) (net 18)))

